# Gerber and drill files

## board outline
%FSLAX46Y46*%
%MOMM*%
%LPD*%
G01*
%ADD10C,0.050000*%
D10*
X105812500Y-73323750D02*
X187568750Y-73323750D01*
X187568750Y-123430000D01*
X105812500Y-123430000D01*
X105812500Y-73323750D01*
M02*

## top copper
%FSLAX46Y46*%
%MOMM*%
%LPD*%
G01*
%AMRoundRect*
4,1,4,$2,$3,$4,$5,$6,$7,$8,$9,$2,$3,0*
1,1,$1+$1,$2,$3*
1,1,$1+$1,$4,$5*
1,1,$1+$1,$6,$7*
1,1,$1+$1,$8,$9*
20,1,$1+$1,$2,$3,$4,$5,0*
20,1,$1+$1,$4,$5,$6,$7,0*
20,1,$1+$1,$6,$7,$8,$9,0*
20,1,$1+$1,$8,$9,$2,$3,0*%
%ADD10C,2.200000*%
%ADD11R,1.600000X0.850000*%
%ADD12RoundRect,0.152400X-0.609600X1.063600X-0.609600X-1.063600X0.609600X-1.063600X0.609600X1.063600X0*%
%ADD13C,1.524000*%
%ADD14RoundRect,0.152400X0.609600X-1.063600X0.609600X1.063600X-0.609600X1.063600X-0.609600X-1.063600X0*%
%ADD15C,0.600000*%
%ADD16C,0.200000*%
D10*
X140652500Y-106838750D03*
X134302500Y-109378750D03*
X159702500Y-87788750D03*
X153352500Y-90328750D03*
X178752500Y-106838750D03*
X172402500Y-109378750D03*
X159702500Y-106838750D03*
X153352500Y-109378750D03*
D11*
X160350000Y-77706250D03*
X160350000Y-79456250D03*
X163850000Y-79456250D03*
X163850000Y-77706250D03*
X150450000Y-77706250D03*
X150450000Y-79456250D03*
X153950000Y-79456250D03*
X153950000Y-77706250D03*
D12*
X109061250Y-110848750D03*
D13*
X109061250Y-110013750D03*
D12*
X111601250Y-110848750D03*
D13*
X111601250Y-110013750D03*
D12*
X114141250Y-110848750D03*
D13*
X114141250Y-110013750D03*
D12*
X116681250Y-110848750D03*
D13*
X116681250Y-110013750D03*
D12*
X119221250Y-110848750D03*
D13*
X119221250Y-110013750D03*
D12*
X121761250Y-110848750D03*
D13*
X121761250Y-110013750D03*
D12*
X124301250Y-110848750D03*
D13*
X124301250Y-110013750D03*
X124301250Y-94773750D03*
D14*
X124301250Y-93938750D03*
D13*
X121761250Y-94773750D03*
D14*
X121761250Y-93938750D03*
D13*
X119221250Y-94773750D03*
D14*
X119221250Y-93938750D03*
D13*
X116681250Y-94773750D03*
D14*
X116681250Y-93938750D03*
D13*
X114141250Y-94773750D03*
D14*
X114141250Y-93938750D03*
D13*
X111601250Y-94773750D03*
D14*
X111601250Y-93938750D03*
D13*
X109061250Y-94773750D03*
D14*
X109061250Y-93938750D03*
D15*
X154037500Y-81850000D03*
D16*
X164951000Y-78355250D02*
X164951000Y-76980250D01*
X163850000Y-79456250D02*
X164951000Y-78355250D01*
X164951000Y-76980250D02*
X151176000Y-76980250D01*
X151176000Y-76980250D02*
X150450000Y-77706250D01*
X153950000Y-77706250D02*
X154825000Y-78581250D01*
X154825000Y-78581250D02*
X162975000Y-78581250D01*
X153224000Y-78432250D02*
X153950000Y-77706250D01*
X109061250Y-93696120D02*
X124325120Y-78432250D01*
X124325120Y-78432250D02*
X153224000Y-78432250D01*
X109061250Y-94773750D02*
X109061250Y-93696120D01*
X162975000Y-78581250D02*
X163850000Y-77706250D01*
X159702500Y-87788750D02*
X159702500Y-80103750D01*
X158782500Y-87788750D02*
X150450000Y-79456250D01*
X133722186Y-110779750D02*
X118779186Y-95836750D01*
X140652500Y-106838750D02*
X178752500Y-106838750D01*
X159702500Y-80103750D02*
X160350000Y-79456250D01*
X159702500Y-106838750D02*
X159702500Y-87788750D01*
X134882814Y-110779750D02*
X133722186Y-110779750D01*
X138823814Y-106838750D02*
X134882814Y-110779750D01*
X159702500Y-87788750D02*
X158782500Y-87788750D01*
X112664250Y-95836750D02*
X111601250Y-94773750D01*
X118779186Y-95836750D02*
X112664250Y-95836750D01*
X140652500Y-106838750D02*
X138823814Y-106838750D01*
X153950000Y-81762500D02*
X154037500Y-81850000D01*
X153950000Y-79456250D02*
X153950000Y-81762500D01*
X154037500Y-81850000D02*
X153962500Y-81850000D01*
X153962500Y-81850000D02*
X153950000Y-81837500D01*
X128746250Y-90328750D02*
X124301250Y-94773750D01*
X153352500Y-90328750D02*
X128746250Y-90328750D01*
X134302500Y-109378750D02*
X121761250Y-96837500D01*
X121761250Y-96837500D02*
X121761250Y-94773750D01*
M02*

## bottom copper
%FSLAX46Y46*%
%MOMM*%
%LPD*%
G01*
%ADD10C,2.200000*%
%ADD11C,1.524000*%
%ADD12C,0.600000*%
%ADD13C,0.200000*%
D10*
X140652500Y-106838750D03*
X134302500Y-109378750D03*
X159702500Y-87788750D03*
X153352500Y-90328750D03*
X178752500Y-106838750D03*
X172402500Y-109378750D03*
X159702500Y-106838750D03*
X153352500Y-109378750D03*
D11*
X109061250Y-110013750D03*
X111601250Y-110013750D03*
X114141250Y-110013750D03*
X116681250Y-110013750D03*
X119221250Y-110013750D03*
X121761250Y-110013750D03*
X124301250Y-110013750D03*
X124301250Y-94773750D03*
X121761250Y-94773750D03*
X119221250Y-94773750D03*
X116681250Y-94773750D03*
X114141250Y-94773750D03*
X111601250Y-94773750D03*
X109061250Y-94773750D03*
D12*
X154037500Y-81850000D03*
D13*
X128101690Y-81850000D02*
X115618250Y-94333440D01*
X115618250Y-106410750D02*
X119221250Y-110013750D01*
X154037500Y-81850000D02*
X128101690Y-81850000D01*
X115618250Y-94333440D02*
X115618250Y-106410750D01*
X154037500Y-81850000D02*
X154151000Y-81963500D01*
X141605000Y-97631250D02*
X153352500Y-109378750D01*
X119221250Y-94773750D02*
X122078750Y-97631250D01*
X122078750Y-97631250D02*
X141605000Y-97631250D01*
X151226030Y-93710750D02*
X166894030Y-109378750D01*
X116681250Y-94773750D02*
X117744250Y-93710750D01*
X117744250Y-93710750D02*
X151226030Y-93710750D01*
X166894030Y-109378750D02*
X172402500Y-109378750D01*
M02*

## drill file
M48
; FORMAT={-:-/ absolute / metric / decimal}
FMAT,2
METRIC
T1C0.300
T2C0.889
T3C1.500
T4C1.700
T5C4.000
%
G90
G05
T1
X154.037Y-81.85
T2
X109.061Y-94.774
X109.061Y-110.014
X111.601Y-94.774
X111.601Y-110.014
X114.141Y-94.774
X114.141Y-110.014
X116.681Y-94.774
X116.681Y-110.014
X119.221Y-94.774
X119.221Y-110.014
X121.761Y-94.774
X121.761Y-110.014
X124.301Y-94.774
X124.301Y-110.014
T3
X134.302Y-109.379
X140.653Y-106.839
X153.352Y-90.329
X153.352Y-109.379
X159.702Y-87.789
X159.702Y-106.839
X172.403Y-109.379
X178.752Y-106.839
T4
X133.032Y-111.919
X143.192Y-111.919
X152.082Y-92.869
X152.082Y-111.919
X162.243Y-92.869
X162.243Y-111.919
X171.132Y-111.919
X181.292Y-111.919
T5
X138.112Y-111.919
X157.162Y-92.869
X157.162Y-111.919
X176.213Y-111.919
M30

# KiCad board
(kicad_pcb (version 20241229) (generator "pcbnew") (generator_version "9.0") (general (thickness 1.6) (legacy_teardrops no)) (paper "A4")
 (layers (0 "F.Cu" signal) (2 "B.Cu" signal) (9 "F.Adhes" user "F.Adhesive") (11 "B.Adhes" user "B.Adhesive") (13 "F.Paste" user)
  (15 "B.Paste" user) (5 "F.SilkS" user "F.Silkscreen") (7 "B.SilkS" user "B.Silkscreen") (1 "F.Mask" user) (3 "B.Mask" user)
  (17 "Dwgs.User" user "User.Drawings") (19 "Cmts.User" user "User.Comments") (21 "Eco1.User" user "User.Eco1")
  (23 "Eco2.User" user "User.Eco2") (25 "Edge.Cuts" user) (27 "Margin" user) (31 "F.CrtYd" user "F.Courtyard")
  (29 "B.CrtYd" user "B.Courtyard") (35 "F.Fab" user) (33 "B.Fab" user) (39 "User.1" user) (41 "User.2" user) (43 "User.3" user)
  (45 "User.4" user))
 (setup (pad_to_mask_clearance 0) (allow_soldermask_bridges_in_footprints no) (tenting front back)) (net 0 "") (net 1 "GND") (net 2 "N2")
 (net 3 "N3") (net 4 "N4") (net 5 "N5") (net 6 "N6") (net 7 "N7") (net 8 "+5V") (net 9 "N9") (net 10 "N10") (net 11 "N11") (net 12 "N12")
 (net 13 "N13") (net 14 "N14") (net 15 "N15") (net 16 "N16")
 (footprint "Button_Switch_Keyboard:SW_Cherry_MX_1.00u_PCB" (layer "F.Cu") (at 140.6525 106.83875)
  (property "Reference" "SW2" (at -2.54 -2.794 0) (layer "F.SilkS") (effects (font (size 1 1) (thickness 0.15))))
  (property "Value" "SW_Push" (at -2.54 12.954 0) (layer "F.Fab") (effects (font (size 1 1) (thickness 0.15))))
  (pad "" np_thru_hole circle (at -7.62 5.08) (size 1.7 1.7) (drill 1.7) (layers "*.Cu" "*.Mask"))
  (pad "" np_thru_hole circle (at -2.54 5.08) (size 4 4) (drill 4) (layers "*.Cu" "*.Mask"))
  (pad "" np_thru_hole circle (at 2.54 5.08) (size 1.7 1.7) (drill 1.7) (layers "*.Cu" "*.Mask"))
  (pad "1" thru_hole circle (at 0 0) (size 2.2 2.2) (drill 1.5) (layers "*.Cu" "*.Mask") (remove_unused_layers no) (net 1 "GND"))
  (pad "2" thru_hole circle (at -6.35 2.54) (size 2.2 2.2) (drill 1.5) (layers "*.Cu" "*.Mask") (remove_unused_layers no) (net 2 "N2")))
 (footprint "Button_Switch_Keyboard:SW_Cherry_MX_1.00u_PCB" (layer "F.Cu") (at 159.7025 87.78875)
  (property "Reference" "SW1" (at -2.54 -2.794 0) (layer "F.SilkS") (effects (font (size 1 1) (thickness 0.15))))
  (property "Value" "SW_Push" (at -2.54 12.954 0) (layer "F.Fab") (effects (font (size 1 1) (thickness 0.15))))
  (pad "" np_thru_hole circle (at -7.62 5.08) (size 1.7 1.7) (drill 1.7) (layers "*.Cu" "*.Mask"))
  (pad "" np_thru_hole circle (at -2.54 5.08) (size 4 4) (drill 4) (layers "*.Cu" "*.Mask"))
  (pad "" np_thru_hole circle (at 2.54 5.08) (size 1.7 1.7) (drill 1.7) (layers "*.Cu" "*.Mask"))
  (pad "1" thru_hole circle (at 0 0) (size 2.2 2.2) (drill 1.5) (layers "*.Cu" "*.Mask") (remove_unused_layers no) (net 1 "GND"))
  (pad "2" thru_hole circle (at -6.35 2.54) (size 2.2 2.2) (drill 1.5) (layers "*.Cu" "*.Mask") (remove_unused_layers no) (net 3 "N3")))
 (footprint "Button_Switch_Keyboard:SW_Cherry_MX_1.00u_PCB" (layer "F.Cu") (at 178.7525 106.83875)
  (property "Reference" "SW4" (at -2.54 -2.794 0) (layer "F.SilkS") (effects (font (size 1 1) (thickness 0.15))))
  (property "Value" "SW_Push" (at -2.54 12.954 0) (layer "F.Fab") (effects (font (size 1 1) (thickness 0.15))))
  (pad "" np_thru_hole circle (at -7.62 5.08) (size 1.7 1.7) (drill 1.7) (layers "*.Cu" "*.Mask"))
  (pad "" np_thru_hole circle (at -2.54 5.08) (size 4 4) (drill 4) (layers "*.Cu" "*.Mask"))
  (pad "" np_thru_hole circle (at 2.54 5.08) (size 1.7 1.7) (drill 1.7) (layers "*.Cu" "*.Mask"))
  (pad "1" thru_hole circle (at 0 0) (size 2.2 2.2) (drill 1.5) (layers "*.Cu" "*.Mask") (remove_unused_layers no) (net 1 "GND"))
  (pad "2" thru_hole circle (at -6.35 2.54) (size 2.2 2.2) (drill 1.5) (layers "*.Cu" "*.Mask") (remove_unused_layers no) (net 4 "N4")))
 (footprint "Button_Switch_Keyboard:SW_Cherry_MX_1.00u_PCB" (layer "F.Cu") (at 159.7025 106.83875)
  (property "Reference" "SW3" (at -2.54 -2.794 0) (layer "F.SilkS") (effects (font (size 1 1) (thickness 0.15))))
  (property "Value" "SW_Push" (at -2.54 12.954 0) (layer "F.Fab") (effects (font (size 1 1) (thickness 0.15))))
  (pad "" np_thru_hole circle (at -7.62 5.08) (size 1.7 1.7) (drill 1.7) (layers "*.Cu" "*.Mask"))
  (pad "" np_thru_hole circle (at -2.54 5.08) (size 4 4) (drill 4) (layers "*.Cu" "*.Mask"))
  (pad "" np_thru_hole circle (at 2.54 5.08) (size 1.7 1.7) (drill 1.7) (layers "*.Cu" "*.Mask"))
  (pad "1" thru_hole circle (at 0 0) (size 2.2 2.2) (drill 1.5) (layers "*.Cu" "*.Mask") (remove_unused_layers no) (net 1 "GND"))
  (pad "2" thru_hole circle (at -6.35 2.54) (size 2.2 2.2) (drill 1.5) (layers "*.Cu" "*.Mask") (remove_unused_layers no) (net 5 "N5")))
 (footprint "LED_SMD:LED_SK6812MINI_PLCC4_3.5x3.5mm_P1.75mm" (layer "F.Cu") (at 162.1 78.58125)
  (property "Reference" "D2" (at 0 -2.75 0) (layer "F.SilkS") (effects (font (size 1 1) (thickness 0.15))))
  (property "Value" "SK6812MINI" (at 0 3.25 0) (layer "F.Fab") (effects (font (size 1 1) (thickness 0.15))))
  (pad "1" smd rect (at -1.75 -0.875) (size 1.6 0.85) (layers "F.Cu" "F.Mask" "F.Paste") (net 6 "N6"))
  (pad "2" smd rect (at -1.75 0.875) (size 1.6 0.85) (layers "F.Cu" "F.Mask" "F.Paste") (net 1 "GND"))
  (pad "3" smd rect (at 1.75 0.875) (size 1.6 0.85) (layers "F.Cu" "F.Mask" "F.Paste") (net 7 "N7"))
  (pad "4" smd rect (at 1.75 -0.875) (size 1.6 0.85) (layers "F.Cu" "F.Mask" "F.Paste") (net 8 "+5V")))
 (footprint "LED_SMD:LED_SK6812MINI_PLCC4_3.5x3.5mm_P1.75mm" (layer "F.Cu") (at 152.2 78.58125)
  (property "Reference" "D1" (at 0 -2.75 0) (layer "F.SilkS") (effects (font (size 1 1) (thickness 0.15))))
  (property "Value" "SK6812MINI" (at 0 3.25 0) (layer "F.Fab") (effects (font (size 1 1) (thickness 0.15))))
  (pad "1" smd rect (at -1.75 -0.875) (size 1.6 0.85) (layers "F.Cu" "F.Mask" "F.Paste") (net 7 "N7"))
  (pad "2" smd rect (at -1.75 0.875) (size 1.6 0.85) (layers "F.Cu" "F.Mask" "F.Paste") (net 1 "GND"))
  (pad "3" smd rect (at 1.75 0.875) (size 1.6 0.85) (layers "F.Cu" "F.Mask" "F.Paste") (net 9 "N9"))
  (pad "4" smd rect (at 1.75 -0.875) (size 1.6 0.85) (layers "F.Cu" "F.Mask" "F.Paste") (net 8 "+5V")))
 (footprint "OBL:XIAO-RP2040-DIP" (layer "F.Cu") (at 116.68125 102.39375 90)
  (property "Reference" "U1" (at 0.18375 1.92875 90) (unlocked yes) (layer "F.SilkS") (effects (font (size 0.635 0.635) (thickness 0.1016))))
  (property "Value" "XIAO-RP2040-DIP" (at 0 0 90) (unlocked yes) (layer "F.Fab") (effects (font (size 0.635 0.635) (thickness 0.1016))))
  (pad "1" smd roundrect (at -8.455 -7.62 270) (size 2.432 1.524) (layers "F.Cu" "F.Mask") (roundrect_rratio 0.1) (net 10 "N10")
   (thermal_bridge_angle 45))
  (pad "1" thru_hole circle (at -7.62 -7.62 270) (size 1.524 1.524) (drill 0.889) (layers "*.Cu" "*.Mask") (remove_unused_layers no)
   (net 10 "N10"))
  (pad "2" smd roundrect (at -8.455 -5.08 270) (size 2.432 1.524) (layers "F.Cu" "F.Mask") (roundrect_rratio 0.1) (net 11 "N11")
   (thermal_bridge_angle 45))
  (pad "2" thru_hole circle (at -7.62 -5.08 270) (size 1.524 1.524) (drill 0.889) (layers "*.Cu" "*.Mask") (remove_unused_layers no)
   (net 11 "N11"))
  (pad "3" smd roundrect (at -8.455 -2.54 270) (size 2.432 1.524) (layers "F.Cu" "F.Mask") (roundrect_rratio 0.1) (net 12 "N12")
   (thermal_bridge_angle 45))
  (pad "3" thru_hole circle (at -7.62 -2.54 270) (size 1.524 1.524) (drill 0.889) (layers "*.Cu" "*.Mask") (remove_unused_layers no)
   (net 12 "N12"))
  (pad "4" smd roundrect (at -8.455 0 270) (size 2.432 1.524) (layers "F.Cu" "F.Mask") (roundrect_rratio 0.1) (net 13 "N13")
   (thermal_bridge_angle 45))
  (pad "4" thru_hole circle (at -7.62 0 270) (size 1.524 1.524) (drill 0.889) (layers "*.Cu" "*.Mask") (remove_unused_layers no)
   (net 13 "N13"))
  (pad "5" smd roundrect (at -8.455 2.54 270) (size 2.432 1.524) (layers "F.Cu" "F.Mask") (roundrect_rratio 0.1) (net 9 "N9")
   (thermal_bridge_angle 45))
  (pad "5" thru_hole circle (at -7.62 2.54 270) (size 1.524 1.524) (drill 0.889) (layers "*.Cu" "*.Mask") (remove_unused_layers no)
   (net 9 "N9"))
  (pad "6" smd roundrect (at -8.455 5.08 270) (size 2.432 1.524) (layers "F.Cu" "F.Mask") (roundrect_rratio 0.1) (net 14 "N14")
   (thermal_bridge_angle 45))
  (pad "6" thru_hole circle (at -7.62 5.08 270) (size 1.524 1.524) (drill 0.889) (layers "*.Cu" "*.Mask") (remove_unused_layers no)
   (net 14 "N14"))
  (pad "7" smd roundrect (at -8.455 7.62 270) (size 2.432 1.524) (layers "F.Cu" "F.Mask") (roundrect_rratio 0.1) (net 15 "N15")
   (thermal_bridge_angle 45))
  (pad "7" thru_hole circle (at -7.62 7.62 270) (size 1.524 1.524) (drill 0.889) (layers "*.Cu" "*.Mask") (remove_unused_layers no)
   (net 15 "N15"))
  (pad "8" thru_hole circle (at 7.62 7.62 90) (size 1.524 1.524) (drill 0.889) (layers "*.Cu" "*.Mask") (remove_unused_layers no)
   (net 3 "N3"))
  (pad "8" smd roundrect (at 8.455 7.62 90) (size 2.432 1.524) (layers "F.Cu" "F.Mask") (roundrect_rratio 0.1) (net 3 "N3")
   (thermal_bridge_angle 45))
  (pad "9" thru_hole circle (at 7.62 5.08 90) (size 1.524 1.524) (drill 0.889) (layers "*.Cu" "*.Mask") (remove_unused_layers no)
   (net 2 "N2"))
  (pad "9" smd roundrect (at 8.455 5.08 90) (size 2.432 1.524) (layers "F.Cu" "F.Mask") (roundrect_rratio 0.1) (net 2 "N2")
   (thermal_bridge_angle 45))
  (pad "10" thru_hole circle (at 7.62 2.54 90) (size 1.524 1.524) (drill 0.889) (layers "*.Cu" "*.Mask") (remove_unused_layers no)
   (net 5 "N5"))
  (pad "10" smd roundrect (at 8.455 2.54 90) (size 2.432 1.524) (layers "F.Cu" "F.Mask") (roundrect_rratio 0.1) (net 5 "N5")
   (thermal_bridge_angle 45))
  (pad "11" thru_hole circle (at 7.62 0 90) (size 1.524 1.524) (drill 0.889) (layers "*.Cu" "*.Mask") (remove_unused_layers no) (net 4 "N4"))
  (pad "11" smd roundrect (at 8.455 0 90) (size 2.432 1.524) (layers "F.Cu" "F.Mask") (roundrect_rratio 0.1) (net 4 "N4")
   (thermal_bridge_angle 45))
  (pad "12" thru_hole circle (at 7.62 -2.54 90) (size 1.524 1.524) (drill 0.889) (layers "*.Cu" "*.Mask") (remove_unused_layers no)
   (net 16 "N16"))
  (pad "12" smd roundrect (at 8.455 -2.54 90) (size 2.432 1.524) (layers "F.Cu" "F.Mask") (roundrect_rratio 0.1) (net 16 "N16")
   (thermal_bridge_angle 45))
  (pad "13" thru_hole circle (at 7.62 -5.08 90) (size 1.524 1.524) (drill 0.889) (layers "*.Cu" "*.Mask") (remove_unused_layers no)
   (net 1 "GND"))
  (pad "13" smd roundrect (at 8.455 -5.08 90) (size 2.432 1.524) (layers "F.Cu" "F.Mask") (roundrect_rratio 0.1) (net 1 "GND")
   (thermal_bridge_angle 45))
  (pad "14" thru_hole circle (at 7.62 -7.62 90) (size 1.524 1.524) (drill 0.889) (layers "*.Cu" "*.Mask") (remove_unused_layers no)
   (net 8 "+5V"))
  (pad "14" smd roundrect (at 8.455 -7.62 90) (size 2.432 1.524) (layers "F.Cu" "F.Mask") (roundrect_rratio 0.1) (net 8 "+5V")
   (thermal_bridge_angle 45)))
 (gr_rect (start 105.8125 73.32375) (end 187.56875 123.43) (stroke (width 0.05) (type solid)) (fill no) (layer "Edge.Cuts"))
 (segment (start 164.951 78.35525) (end 164.951 76.98025) (width 0.2) (layer "F.Cu") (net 7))
 (segment (start 163.85 79.45625) (end 164.951 78.35525) (width 0.2) (layer "F.Cu") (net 7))
 (segment (start 164.951 76.98025) (end 151.176 76.98025) (width 0.2) (layer "F.Cu") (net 7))
 (segment (start 151.176 76.98025) (end 150.45 77.70625) (width 0.2) (layer "F.Cu") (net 7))
 (segment (start 153.95 77.70625) (end 154.825 78.58125) (width 0.2) (layer "F.Cu") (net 8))
 (segment (start 154.825 78.58125) (end 162.975 78.58125) (width 0.2) (layer "F.Cu") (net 8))
 (segment (start 153.224 78.43225) (end 153.95 77.70625) (width 0.2) (layer "F.Cu") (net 8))
 (segment (start 109.06125 93.69612) (end 124.32512 78.43225) (width 0.2) (layer "F.Cu") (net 8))
 (segment (start 124.32512 78.43225) (end 153.224 78.43225) (width 0.2) (layer "F.Cu") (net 8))
 (segment (start 109.06125 94.77375) (end 109.06125 93.69612) (width 0.2) (layer "F.Cu") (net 8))
 (segment (start 162.975 78.58125) (end 163.85 77.70625) (width 0.2) (layer "F.Cu") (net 8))
 (segment (start 159.7025 87.78875) (end 159.7025 80.10375) (width 0.2) (layer "F.Cu") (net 1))
 (segment (start 158.7825 87.78875) (end 150.45 79.45625) (width 0.2) (layer "F.Cu") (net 1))
 (segment (start 133.722186 110.77975) (end 118.779186 95.83675) (width 0.2) (layer "F.Cu") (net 1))
 (segment (start 140.6525 106.83875) (end 178.7525 106.83875) (width 0.2) (layer "F.Cu") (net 1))
 (segment (start 159.7025 80.10375) (end 160.35 79.45625) (width 0.2) (layer "F.Cu") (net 1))
 (segment (start 159.7025 106.83875) (end 159.7025 87.78875) (width 0.2) (layer "F.Cu") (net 1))
 (segment (start 134.882814 110.77975) (end 133.722186 110.77975) (width 0.2) (layer "F.Cu") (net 1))
 (segment (start 138.823814 106.83875) (end 134.882814 110.77975) (width 0.2) (layer "F.Cu") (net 1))
 (segment (start 159.7025 87.78875) (end 158.7825 87.78875) (width 0.2) (layer "F.Cu") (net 1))
 (segment (start 112.66425 95.83675) (end 111.60125 94.77375) (width 0.2) (layer "F.Cu") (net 1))
 (segment (start 118.779186 95.83675) (end 112.66425 95.83675) (width 0.2) (layer "F.Cu") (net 1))
 (segment (start 140.6525 106.83875) (end 138.823814 106.83875) (width 0.2) (layer "F.Cu") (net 1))
 (segment (start 153.95 81.7625) (end 154.0375 81.85) (width 0.2) (layer "F.Cu") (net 9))
 (segment (start 153.95 79.45625) (end 153.95 81.7625) (width 0.2) (layer "F.Cu") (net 9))
 (segment (start 154.0375 81.85) (end 153.9625 81.85) (width 0.2) (layer "F.Cu") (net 9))
 (segment (start 153.9625 81.85) (end 153.95 81.8375) (width 0.2) (layer "F.Cu") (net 9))
 (via (at 154.0375 81.85) (size 0.6) (drill 0.3) (layers "F.Cu" "B.Cu") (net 9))
 (segment (start 128.10169 81.85) (end 115.61825 94.33344) (width 0.2) (layer "B.Cu") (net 9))
 (segment (start 115.61825 106.41075) (end 119.22125 110.01375) (width 0.2) (layer "B.Cu") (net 9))
 (segment (start 154.0375 81.85) (end 128.10169 81.85) (width 0.2) (layer "B.Cu") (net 9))
 (segment (start 115.61825 94.33344) (end 115.61825 106.41075) (width 0.2) (layer "B.Cu") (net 9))
 (segment (start 154.0375 81.85) (end 154.151 81.9635) (width 0.2) (layer "B.Cu") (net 9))
 (segment (start 128.74625 90.32875) (end 124.30125 94.77375) (width 0.2) (layer "F.Cu") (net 3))
 (segment (start 153.3525 90.32875) (end 128.74625 90.32875) (width 0.2) (layer "F.Cu") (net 3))
 (segment (start 134.3025 109.37875) (end 121.76125 96.8375) (width 0.2) (layer "F.Cu") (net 2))
 (segment (start 121.76125 96.8375) (end 121.76125 94.77375) (width 0.2) (layer "F.Cu") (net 2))
 (segment (start 141.605 97.63125) (end 153.3525 109.37875) (width 0.2) (layer "B.Cu") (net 5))
 (segment (start 119.22125 94.77375) (end 122.07875 97.63125) (width 0.2) (layer "B.Cu") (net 5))
 (segment (start 122.07875 97.63125) (end 141.605 97.63125) (width 0.2) (layer "B.Cu") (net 5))
 (segment (start 151.22603 93.71075) (end 166.89403 109.37875) (width 0.2) (layer "B.Cu") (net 4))
 (segment (start 116.68125 94.77375) (end 117.74425 93.71075) (width 0.2) (layer "B.Cu") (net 4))
 (segment (start 117.74425 93.71075) (end 151.22603 93.71075) (width 0.2) (layer "B.Cu") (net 4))
 (segment (start 166.89403 109.37875) (end 172.4025 109.37875) (width 0.2) (layer "B.Cu") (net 4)))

